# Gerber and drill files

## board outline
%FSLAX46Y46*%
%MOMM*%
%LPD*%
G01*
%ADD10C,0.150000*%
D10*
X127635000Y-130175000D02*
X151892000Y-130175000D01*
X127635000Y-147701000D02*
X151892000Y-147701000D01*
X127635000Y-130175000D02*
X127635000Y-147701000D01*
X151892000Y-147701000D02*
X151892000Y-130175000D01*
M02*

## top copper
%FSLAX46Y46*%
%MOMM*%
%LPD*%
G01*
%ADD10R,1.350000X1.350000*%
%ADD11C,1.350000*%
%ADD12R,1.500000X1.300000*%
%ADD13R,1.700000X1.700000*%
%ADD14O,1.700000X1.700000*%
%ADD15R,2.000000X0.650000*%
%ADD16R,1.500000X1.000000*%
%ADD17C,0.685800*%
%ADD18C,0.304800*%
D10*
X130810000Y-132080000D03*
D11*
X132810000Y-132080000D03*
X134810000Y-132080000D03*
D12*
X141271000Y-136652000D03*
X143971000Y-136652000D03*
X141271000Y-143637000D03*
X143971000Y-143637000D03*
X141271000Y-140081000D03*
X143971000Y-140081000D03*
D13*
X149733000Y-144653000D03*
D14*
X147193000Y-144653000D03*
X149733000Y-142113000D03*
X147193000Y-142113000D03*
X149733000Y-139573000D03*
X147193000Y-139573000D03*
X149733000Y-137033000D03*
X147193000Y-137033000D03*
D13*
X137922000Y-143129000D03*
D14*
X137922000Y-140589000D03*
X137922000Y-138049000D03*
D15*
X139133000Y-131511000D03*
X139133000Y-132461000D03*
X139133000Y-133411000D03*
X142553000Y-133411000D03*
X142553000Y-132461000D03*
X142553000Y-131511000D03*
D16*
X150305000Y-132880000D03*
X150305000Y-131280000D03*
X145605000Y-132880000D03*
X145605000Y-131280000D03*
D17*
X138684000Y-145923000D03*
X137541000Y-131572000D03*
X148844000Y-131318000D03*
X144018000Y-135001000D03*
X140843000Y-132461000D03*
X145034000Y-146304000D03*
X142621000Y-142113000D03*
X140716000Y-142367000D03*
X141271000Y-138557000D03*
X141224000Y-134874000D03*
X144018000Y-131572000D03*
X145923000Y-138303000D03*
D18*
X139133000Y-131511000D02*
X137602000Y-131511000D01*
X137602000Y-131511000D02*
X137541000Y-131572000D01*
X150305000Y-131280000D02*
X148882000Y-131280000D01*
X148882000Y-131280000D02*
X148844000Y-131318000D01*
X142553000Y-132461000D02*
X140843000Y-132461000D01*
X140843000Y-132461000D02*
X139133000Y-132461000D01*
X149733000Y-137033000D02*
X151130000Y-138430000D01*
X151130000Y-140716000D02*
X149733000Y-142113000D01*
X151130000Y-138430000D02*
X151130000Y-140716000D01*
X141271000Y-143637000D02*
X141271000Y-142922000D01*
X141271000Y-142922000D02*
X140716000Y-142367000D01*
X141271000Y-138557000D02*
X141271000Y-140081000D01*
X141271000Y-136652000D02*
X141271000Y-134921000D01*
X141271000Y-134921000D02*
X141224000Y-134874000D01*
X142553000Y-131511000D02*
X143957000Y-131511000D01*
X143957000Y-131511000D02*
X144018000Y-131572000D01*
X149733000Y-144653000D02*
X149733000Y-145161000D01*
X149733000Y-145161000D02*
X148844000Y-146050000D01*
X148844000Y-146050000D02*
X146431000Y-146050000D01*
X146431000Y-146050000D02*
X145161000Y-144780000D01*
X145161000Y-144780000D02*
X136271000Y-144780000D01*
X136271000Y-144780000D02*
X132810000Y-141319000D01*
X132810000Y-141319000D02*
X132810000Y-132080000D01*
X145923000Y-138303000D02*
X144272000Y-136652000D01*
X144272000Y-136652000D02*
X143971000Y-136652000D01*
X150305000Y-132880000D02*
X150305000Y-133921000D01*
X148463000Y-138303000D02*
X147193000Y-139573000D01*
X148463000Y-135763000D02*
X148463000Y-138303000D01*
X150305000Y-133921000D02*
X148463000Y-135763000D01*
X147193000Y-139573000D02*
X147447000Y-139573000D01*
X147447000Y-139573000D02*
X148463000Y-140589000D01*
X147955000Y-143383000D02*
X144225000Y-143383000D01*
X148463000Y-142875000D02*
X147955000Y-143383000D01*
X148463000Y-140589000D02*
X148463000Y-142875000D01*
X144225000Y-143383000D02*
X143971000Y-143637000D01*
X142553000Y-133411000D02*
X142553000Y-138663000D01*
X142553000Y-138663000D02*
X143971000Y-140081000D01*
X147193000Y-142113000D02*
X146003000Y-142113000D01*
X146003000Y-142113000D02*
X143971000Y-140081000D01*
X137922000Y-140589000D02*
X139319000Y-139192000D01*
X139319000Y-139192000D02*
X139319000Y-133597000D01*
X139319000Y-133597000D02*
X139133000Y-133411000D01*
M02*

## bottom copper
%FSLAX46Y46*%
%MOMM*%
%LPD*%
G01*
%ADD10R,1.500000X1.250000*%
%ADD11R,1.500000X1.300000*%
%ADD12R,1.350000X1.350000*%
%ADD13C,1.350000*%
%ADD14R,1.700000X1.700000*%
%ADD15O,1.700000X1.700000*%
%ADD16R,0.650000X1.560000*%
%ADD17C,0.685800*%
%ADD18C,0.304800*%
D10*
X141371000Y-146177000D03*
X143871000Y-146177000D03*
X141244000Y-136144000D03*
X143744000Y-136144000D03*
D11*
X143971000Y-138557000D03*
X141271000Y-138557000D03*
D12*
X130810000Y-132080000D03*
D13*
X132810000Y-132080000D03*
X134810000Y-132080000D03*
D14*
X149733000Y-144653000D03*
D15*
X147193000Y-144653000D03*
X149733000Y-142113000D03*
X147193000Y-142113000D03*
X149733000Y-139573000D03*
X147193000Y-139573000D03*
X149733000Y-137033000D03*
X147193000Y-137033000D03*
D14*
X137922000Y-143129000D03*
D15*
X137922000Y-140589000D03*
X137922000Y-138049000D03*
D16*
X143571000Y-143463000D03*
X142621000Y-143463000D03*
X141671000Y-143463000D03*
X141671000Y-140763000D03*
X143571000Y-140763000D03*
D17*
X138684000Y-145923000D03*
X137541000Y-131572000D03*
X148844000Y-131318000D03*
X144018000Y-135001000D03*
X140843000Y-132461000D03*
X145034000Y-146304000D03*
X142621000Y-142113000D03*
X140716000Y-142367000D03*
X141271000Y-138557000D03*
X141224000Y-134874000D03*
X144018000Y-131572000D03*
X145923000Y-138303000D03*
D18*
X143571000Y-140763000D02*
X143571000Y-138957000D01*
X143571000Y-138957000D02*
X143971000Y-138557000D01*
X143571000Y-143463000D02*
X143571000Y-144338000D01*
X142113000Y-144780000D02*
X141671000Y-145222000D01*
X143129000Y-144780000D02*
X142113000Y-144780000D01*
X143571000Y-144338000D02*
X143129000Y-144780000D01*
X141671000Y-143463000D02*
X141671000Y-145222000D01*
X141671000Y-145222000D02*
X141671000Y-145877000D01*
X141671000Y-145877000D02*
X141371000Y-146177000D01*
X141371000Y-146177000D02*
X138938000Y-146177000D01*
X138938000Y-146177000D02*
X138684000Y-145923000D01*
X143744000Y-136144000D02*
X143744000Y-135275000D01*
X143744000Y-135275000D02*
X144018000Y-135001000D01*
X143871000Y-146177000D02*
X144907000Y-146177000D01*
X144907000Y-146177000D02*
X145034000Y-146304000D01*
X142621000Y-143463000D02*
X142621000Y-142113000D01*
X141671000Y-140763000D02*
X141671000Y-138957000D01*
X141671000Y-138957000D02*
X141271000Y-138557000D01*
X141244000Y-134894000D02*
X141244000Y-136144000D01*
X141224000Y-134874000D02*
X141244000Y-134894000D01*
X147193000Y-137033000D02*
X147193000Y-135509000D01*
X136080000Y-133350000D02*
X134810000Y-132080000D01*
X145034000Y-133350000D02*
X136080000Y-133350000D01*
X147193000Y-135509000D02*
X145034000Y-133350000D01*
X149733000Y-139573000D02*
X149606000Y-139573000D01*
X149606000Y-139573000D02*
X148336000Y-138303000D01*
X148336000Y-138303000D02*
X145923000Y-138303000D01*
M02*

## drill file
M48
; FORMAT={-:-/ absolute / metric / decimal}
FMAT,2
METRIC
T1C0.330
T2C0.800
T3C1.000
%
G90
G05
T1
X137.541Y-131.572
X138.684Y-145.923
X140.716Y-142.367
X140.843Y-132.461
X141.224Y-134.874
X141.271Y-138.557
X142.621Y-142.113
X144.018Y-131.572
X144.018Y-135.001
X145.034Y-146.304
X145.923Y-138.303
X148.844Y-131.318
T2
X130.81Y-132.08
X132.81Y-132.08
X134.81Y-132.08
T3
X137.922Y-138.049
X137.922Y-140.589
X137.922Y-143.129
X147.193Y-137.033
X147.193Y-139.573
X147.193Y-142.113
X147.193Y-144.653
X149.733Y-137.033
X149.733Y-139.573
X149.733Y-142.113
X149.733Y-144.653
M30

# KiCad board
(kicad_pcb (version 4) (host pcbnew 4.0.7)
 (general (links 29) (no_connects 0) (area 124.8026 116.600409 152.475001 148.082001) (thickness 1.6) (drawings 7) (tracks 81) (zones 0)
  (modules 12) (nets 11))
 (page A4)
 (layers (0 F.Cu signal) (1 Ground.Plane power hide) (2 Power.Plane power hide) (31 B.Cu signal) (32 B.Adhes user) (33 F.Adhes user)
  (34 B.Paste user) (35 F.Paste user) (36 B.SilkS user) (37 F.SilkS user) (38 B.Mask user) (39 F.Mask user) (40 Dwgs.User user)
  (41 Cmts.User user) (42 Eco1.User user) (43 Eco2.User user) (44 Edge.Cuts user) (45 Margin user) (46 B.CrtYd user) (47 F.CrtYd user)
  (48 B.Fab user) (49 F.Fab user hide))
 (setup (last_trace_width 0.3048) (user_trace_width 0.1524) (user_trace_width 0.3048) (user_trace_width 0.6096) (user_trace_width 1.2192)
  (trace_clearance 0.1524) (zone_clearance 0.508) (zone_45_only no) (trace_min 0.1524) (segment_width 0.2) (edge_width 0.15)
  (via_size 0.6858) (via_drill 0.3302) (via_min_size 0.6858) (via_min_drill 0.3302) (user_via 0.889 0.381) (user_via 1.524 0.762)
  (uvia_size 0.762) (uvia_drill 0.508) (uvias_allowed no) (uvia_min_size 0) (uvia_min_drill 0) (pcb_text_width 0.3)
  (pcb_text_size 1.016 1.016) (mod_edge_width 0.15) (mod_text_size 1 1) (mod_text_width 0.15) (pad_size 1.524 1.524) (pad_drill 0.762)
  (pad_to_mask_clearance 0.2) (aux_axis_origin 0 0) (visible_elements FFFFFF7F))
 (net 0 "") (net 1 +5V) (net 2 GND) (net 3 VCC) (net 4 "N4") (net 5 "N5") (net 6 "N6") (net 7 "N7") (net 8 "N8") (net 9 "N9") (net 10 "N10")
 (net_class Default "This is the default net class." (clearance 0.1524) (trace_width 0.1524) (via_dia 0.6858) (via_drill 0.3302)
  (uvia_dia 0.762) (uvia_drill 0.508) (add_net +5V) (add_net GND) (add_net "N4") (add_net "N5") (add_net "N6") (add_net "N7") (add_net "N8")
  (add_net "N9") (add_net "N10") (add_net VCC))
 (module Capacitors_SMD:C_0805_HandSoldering (layer B.Cu) (at 142.621 146.177)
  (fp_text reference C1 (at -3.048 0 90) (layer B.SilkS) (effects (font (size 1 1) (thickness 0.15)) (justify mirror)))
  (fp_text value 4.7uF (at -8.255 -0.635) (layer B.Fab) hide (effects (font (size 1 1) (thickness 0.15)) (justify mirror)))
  (pad 1 smd rect (at -1.25 0) (size 1.5 1.25) (layers B.Cu B.Paste B.Mask) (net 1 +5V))
  (pad 2 smd rect (at 1.25 0) (size 1.5 1.25) (layers B.Cu B.Paste B.Mask) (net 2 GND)))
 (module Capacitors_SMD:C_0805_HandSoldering (layer B.Cu) (at 142.494 136.144)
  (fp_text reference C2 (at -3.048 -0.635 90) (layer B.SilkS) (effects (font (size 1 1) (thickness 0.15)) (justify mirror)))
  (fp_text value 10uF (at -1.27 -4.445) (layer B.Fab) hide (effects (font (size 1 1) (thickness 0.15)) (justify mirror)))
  (pad 1 smd rect (at -1.25 0) (size 1.5 1.25) (layers B.Cu B.Paste B.Mask) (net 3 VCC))
  (pad 2 smd rect (at 1.25 0) (size 1.5 1.25) (layers B.Cu B.Paste B.Mask) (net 2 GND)))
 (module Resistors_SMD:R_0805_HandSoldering (layer B.Cu) (at 142.621 138.557 180)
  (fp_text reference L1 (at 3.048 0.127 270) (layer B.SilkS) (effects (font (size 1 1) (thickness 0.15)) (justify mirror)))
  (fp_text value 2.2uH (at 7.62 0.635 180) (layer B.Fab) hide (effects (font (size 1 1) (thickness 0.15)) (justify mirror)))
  (pad 1 smd rect (at -1.35 0 180) (size 1.5 1.3) (layers B.Cu B.Paste B.Mask) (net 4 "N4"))
  (pad 2 smd rect (at 1.35 0 180) (size 1.5 1.3) (layers B.Cu B.Paste B.Mask) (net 3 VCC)))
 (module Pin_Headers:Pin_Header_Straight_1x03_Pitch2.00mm (layer F.Cu) (at 130.81 132.08 90)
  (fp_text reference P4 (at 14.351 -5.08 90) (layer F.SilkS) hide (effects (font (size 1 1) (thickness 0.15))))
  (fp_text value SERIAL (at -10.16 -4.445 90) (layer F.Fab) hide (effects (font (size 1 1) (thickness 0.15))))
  (pad 1 thru_hole rect (at 0 0 90) (size 1.35 1.35) (drill 0.8) (layers *.Cu *.Mask) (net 2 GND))
  (pad 2 thru_hole circle (at 0 2 90) (size 1.35 1.35) (drill 0.8) (layers *.Cu *.Mask) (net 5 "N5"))
  (pad 3 thru_hole circle (at 0 4 90) (size 1.35 1.35) (drill 0.8) (layers *.Cu *.Mask) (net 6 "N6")))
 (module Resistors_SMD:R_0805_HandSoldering (layer F.Cu) (at 142.621 136.652)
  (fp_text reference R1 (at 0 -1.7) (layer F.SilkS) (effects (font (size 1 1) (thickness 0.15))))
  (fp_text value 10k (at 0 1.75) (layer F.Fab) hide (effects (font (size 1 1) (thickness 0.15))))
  (pad 1 smd rect (at -1.35 0) (size 1.5 1.3) (layers F.Cu F.Paste F.Mask) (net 3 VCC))
  (pad 2 smd rect (at 1.35 0) (size 1.5 1.3) (layers F.Cu F.Paste F.Mask) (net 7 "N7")))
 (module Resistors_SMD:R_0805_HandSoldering (layer F.Cu) (at 142.621 143.637)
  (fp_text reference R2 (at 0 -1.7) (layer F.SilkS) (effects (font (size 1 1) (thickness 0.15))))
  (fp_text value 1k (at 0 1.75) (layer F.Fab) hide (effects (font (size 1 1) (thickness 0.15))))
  (pad 1 smd rect (at -1.35 0) (size 1.5 1.3) (layers F.Cu F.Paste F.Mask) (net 3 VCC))
  (pad 2 smd rect (at 1.35 0) (size 1.5 1.3) (layers F.Cu F.Paste F.Mask) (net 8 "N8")))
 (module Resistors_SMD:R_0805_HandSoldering (layer F.Cu) (at 142.621 140.081)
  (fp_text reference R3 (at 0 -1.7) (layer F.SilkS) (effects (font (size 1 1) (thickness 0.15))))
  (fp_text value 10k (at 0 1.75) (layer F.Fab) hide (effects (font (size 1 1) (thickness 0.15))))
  (pad 1 smd rect (at -1.35 0) (size 1.5 1.3) (layers F.Cu F.Paste F.Mask) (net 3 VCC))
  (pad 2 smd rect (at 1.35 0) (size 1.5 1.3) (layers F.Cu F.Paste F.Mask) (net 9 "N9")))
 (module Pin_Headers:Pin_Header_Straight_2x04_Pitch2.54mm (layer F.Cu) (at 149.733 144.653 180)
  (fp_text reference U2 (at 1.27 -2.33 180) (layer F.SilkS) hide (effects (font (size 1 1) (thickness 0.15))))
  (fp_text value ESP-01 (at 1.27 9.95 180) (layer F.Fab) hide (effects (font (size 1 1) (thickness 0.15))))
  (pad 1 thru_hole rect (at 0 0 180) (size 1.7 1.7) (drill 1) (layers *.Cu *.Mask) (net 5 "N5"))
  (pad 2 thru_hole oval (at 2.54 0 180) (size 1.7 1.7) (drill 1) (layers *.Cu *.Mask) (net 2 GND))
  (pad 3 thru_hole oval (at 0 2.54 180) (size 1.7 1.7) (drill 1) (layers *.Cu *.Mask) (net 3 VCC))
  (pad 4 thru_hole oval (at 2.54 2.54 180) (size 1.7 1.7) (drill 1) (layers *.Cu *.Mask) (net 9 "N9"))
  (pad 5 thru_hole oval (at 0 5.08 180) (size 1.7 1.7) (drill 1) (layers *.Cu *.Mask) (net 7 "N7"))
  (pad 6 thru_hole oval (at 2.54 5.08 180) (size 1.7 1.7) (drill 1) (layers *.Cu *.Mask) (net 8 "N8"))
  (pad 7 thru_hole oval (at 0 7.62 180) (size 1.7 1.7) (drill 1) (layers *.Cu *.Mask) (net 3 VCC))
  (pad 8 thru_hole oval (at 2.54 7.62 180) (size 1.7 1.7) (drill 1) (layers *.Cu *.Mask) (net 6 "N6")))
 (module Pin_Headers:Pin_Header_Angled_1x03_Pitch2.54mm (layer F.Cu) (at 137.922 143.129 180)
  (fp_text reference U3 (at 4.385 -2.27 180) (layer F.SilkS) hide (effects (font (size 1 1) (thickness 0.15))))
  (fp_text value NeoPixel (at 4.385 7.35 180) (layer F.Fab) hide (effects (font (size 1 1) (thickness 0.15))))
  (pad 1 thru_hole rect (at 0 0 180) (size 1.7 1.7) (drill 1) (layers *.Cu *.Mask) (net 2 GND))
  (pad 2 thru_hole oval (at 0 2.54 180) (size 1.7 1.7) (drill 1) (layers *.Cu *.Mask) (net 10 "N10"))
  (pad 3 thru_hole oval (at 0 5.08 180) (size 1.7 1.7) (drill 1) (layers *.Cu *.Mask) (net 1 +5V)))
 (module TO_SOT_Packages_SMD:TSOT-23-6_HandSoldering (layer F.Cu) (at 140.843 132.461)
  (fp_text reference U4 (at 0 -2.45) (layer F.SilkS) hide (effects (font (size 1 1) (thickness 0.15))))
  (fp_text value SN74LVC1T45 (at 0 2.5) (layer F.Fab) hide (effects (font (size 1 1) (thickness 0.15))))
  (pad 1 smd rect (at -1.71 -0.95) (size 2 0.65) (layers F.Cu F.Paste F.Mask) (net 1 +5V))
  (pad 2 smd rect (at -1.71 0) (size 2 0.65) (layers F.Cu F.Paste F.Mask) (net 2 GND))
  (pad 3 smd rect (at -1.71 0.95) (size 2 0.65) (layers F.Cu F.Paste F.Mask) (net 10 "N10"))
  (pad 4 smd rect (at 1.71 0.95) (size 2 0.65) (layers F.Cu F.Paste F.Mask) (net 9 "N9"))
  (pad 5 smd rect (at 1.71 0) (size 2 0.65) (layers F.Cu F.Paste F.Mask) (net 2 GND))
  (pad 6 smd rect (at 1.71 -0.95) (size 2 0.65) (layers F.Cu F.Paste F.Mask) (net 3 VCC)))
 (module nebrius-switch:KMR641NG (layer F.Cu) (at 147.955 132.08 180)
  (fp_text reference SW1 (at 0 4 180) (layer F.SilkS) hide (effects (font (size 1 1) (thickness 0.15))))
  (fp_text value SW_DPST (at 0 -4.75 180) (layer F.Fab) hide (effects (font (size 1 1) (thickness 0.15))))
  (pad 1 smd rect (at -2.35 -0.8 180) (size 1.5 1) (layers F.Cu F.Paste F.Mask) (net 8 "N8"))
  (pad 2 smd rect (at -2.35 0.8 180) (size 1.5 1) (layers F.Cu F.Paste F.Mask) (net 2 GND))
  (pad 3 smd rect (at 2.35 -0.8 180) (size 1.5 1) (layers F.Cu F.Paste F.Mask))
  (pad 4 smd rect (at 2.35 0.8 180) (size 1.5 1) (layers F.Cu F.Paste F.Mask)))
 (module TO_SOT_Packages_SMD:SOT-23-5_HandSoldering (layer B.Cu) (at 142.621 142.113 90)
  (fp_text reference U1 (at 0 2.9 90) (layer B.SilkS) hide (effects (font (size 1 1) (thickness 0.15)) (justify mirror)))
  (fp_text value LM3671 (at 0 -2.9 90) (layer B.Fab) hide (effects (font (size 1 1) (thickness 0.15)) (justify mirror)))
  (pad 1 smd rect (at -1.35 0.95 90) (size 1.56 0.65) (layers B.Cu B.Paste B.Mask) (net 1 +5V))
  (pad 2 smd rect (at -1.35 0 90) (size 1.56 0.65) (layers B.Cu B.Paste B.Mask) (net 2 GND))
  (pad 3 smd rect (at -1.35 -0.95 90) (size 1.56 0.65) (layers B.Cu B.Paste B.Mask) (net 1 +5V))
  (pad 4 smd rect (at 1.35 -0.95 90) (size 1.56 0.65) (layers B.Cu B.Paste B.Mask) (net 3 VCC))
  (pad 5 smd rect (at 1.35 0.95 90) (size 1.56 0.65) (layers B.Cu B.Paste B.Mask) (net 4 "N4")))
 (gr_line (start 127.635 130.175) (end 151.892 130.175) (angle 90) (layer Edge.Cuts) (width 0.15))
 (gr_line (start 127.635 147.701) (end 151.892 147.701) (angle 90) (layer Edge.Cuts) (width 0.15))
 (gr_line (start 127.635 130.175) (end 127.635 147.701) (angle 90) (layer Edge.Cuts) (width 0.15))
 (gr_line (start 151.892 147.701) (end 151.892 130.175) (angle 90) (layer Edge.Cuts) (width 0.15))
 (segment (start 143.571 140.763) (end 143.571 138.957) (width 0.3048) (layer B.Cu) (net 4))
 (segment (start 143.571 138.957) (end 143.971 138.557) (width 0.3048) (layer B.Cu) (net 4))
 (segment (start 143.571 143.463) (end 143.571 144.338) (width 0.3048) (layer B.Cu) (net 1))
 (segment (start 142.113 144.78) (end 141.671 145.222) (width 0.3048) (layer B.Cu) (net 1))
 (segment (start 143.129 144.78) (end 142.113 144.78) (width 0.3048) (layer B.Cu) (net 1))
 (segment (start 143.571 144.338) (end 143.129 144.78) (width 0.3048) (layer B.Cu) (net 1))
 (segment (start 141.671 143.463) (end 141.671 145.222) (width 0.3048) (layer B.Cu) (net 1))
 (segment (start 141.671 145.222) (end 141.671 145.877) (width 0.3048) (layer B.Cu) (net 1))
 (segment (start 141.671 145.877) (end 141.371 146.177) (width 0.3048) (layer B.Cu) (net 1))
 (segment (start 141.371 146.177) (end 138.938 146.177) (width 0.3048) (layer B.Cu) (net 1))
 (via (at 138.684 145.923) (size 0.6858) (drill 0.3302) (layers F.Cu B.Cu) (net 1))
 (segment (start 138.938 146.177) (end 138.684 145.923) (width 0.3048) (layer B.Cu) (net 1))
 (segment (start 139.133 131.511) (end 137.602 131.511) (width 0.3048) (layer F.Cu) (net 1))
 (via (at 137.541 131.572) (size 0.6858) (drill 0.3302) (layers F.Cu B.Cu) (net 1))
 (segment (start 137.602 131.511) (end 137.541 131.572) (width 0.3048) (layer F.Cu) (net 1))
 (segment (start 150.305 131.28) (end 148.882 131.28) (width 0.3048) (layer F.Cu) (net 2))
 (via (at 148.844 131.318) (size 0.6858) (drill 0.3302) (layers F.Cu B.Cu) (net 2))
 (segment (start 148.882 131.28) (end 148.844 131.318) (width 0.3048) (layer F.Cu) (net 2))
 (segment (start 143.744 136.144) (end 143.744 135.275) (width 0.3048) (layer B.Cu) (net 2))
 (via (at 144.018 135.001) (size 0.6858) (drill 0.3302) (layers F.Cu B.Cu) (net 2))
 (segment (start 143.744 135.275) (end 144.018 135.001) (width 0.3048) (layer B.Cu) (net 2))
 (segment (start 142.553 132.461) (end 140.843 132.461) (width 0.3048) (layer F.Cu) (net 2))
 (via (at 140.843 132.461) (size 0.6858) (drill 0.3302) (layers F.Cu B.Cu) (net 2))
 (segment (start 140.843 132.461) (end 139.133 132.461) (width 0.3048) (layer F.Cu) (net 2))
 (segment (start 143.871 146.177) (end 144.907 146.177) (width 0.3048) (layer B.Cu) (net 2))
 (via (at 145.034 146.304) (size 0.6858) (drill 0.3302) (layers F.Cu B.Cu) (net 2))
 (segment (start 144.907 146.177) (end 145.034 146.304) (width 0.3048) (layer B.Cu) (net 2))
 (segment (start 142.621 143.463) (end 142.621 142.113) (width 0.3048) (layer B.Cu) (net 2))
 (via (at 142.621 142.113) (size 0.6858) (drill 0.3302) (layers F.Cu B.Cu) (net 2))
 (segment (start 149.733 137.033) (end 151.13 138.43) (width 0.3048) (layer F.Cu) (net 3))
 (segment (start 151.13 140.716) (end 149.733 142.113) (width 0.3048) (layer F.Cu) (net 3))
 (segment (start 151.13 138.43) (end 151.13 140.716) (width 0.3048) (layer F.Cu) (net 3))
 (segment (start 141.271 143.637) (end 141.271 142.922) (width 0.3048) (layer F.Cu) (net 3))
 (via (at 140.716 142.367) (size 0.6858) (drill 0.3302) (layers F.Cu B.Cu) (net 3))
 (segment (start 141.271 142.922) (end 140.716 142.367) (width 0.3048) (layer F.Cu) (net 3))
 (segment (start 141.671 140.763) (end 141.671 138.957) (width 0.3048) (layer B.Cu) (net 3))
 (segment (start 141.671 138.957) (end 141.271 138.557) (width 0.3048) (layer B.Cu) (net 3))
 (via (at 141.271 138.557) (size 0.6858) (drill 0.3302) (layers F.Cu B.Cu) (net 3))
 (segment (start 141.271 138.557) (end 141.271 140.081) (width 0.3048) (layer F.Cu) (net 3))
 (segment (start 141.271 136.652) (end 141.271 134.921) (width 0.3048) (layer F.Cu) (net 3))
 (segment (start 141.244 134.894) (end 141.244 136.144) (width 0.3048) (layer B.Cu) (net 3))
 (segment (start 141.224 134.874) (end 141.244 134.894) (width 0.3048) (layer B.Cu) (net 3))
 (via (at 141.224 134.874) (size 0.6858) (drill 0.3302) (layers F.Cu B.Cu) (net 3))
 (segment (start 141.271 134.921) (end 141.224 134.874) (width 0.3048) (layer F.Cu) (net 3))
 (segment (start 142.553 131.511) (end 143.957 131.511) (width 0.3048) (layer F.Cu) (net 3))
 (via (at 144.018 131.572) (size 0.6858) (drill 0.3302) (layers F.Cu B.Cu) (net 3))
 (segment (start 143.957 131.511) (end 144.018 131.572) (width 0.3048) (layer F.Cu) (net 3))
 (segment (start 149.733 144.653) (end 149.733 145.161) (width 0.3048) (layer F.Cu) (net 5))
 (segment (start 149.733 145.161) (end 148.844 146.05) (width 0.3048) (layer F.Cu) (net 5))
 (segment (start 148.844 146.05) (end 146.431 146.05) (width 0.3048) (layer F.Cu) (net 5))
 (segment (start 146.431 146.05) (end 145.161 144.78) (width 0.3048) (layer F.Cu) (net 5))
 (segment (start 145.161 144.78) (end 136.271 144.78) (width 0.3048) (layer F.Cu) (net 5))
 (segment (start 136.271 144.78) (end 132.81 141.319) (width 0.3048) (layer F.Cu) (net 5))
 (segment (start 132.81 141.319) (end 132.81 132.08) (width 0.3048) (layer F.Cu) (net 5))
 (segment (start 147.193 137.033) (end 147.193 135.509) (width 0.3048) (layer B.Cu) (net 6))
 (segment (start 136.08 133.35) (end 134.81 132.08) (width 0.3048) (layer B.Cu) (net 6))
 (segment (start 145.034 133.35) (end 136.08 133.35) (width 0.3048) (layer B.Cu) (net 6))
 (segment (start 147.193 135.509) (end 145.034 133.35) (width 0.3048) (layer B.Cu) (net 6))
 (segment (start 149.733 139.573) (end 149.606 139.573) (width 0.3048) (layer B.Cu) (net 7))
 (segment (start 149.606 139.573) (end 148.336 138.303) (width 0.3048) (layer B.Cu) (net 7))
 (segment (start 148.336 138.303) (end 145.923 138.303) (width 0.3048) (layer B.Cu) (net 7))
 (via (at 145.923 138.303) (size 0.6858) (drill 0.3302) (layers F.Cu B.Cu) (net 7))
 (segment (start 145.923 138.303) (end 144.272 136.652) (width 0.3048) (layer F.Cu) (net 7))
 (segment (start 144.272 136.652) (end 143.971 136.652) (width 0.3048) (layer F.Cu) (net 7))
 (segment (start 150.305 132.88) (end 150.305 133.921) (width 0.3048) (layer F.Cu) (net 8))
 (segment (start 148.463 138.303) (end 147.193 139.573) (width 0.3048) (layer F.Cu) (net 8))
 (segment (start 148.463 135.763) (end 148.463 138.303) (width 0.3048) (layer F.Cu) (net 8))
 (segment (start 150.305 133.921) (end 148.463 135.763) (width 0.3048) (layer F.Cu) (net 8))
 (segment (start 147.193 139.573) (end 147.447 139.573) (width 0.3048) (layer F.Cu) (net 8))
 (segment (start 147.447 139.573) (end 148.463 140.589) (width 0.3048) (layer F.Cu) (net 8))
 (segment (start 147.955 143.383) (end 144.225 143.383) (width 0.3048) (layer F.Cu) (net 8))
 (segment (start 148.463 142.875) (end 147.955 143.383) (width 0.3048) (layer F.Cu) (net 8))
 (segment (start 148.463 140.589) (end 148.463 142.875) (width 0.3048) (layer F.Cu) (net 8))
 (segment (start 144.225 143.383) (end 143.971 143.637) (width 0.3048) (layer F.Cu) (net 8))
 (segment (start 142.553 133.411) (end 142.553 138.663) (width 0.3048) (layer F.Cu) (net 9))
 (segment (start 142.553 138.663) (end 143.971 140.081) (width 0.3048) (layer F.Cu) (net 9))
 (segment (start 147.193 142.113) (end 146.003 142.113) (width 0.3048) (layer F.Cu) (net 9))
 (segment (start 146.003 142.113) (end 143.971 140.081) (width 0.3048) (layer F.Cu) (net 9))
 (segment (start 137.922 140.589) (end 139.319 139.192) (width 0.3048) (layer F.Cu) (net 10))
 (segment (start 139.319 139.192) (end 139.319 133.597) (width 0.3048) (layer F.Cu) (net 10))
 (segment (start 139.319 133.597) (end 139.133 133.411) (width 0.3048) (layer F.Cu) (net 10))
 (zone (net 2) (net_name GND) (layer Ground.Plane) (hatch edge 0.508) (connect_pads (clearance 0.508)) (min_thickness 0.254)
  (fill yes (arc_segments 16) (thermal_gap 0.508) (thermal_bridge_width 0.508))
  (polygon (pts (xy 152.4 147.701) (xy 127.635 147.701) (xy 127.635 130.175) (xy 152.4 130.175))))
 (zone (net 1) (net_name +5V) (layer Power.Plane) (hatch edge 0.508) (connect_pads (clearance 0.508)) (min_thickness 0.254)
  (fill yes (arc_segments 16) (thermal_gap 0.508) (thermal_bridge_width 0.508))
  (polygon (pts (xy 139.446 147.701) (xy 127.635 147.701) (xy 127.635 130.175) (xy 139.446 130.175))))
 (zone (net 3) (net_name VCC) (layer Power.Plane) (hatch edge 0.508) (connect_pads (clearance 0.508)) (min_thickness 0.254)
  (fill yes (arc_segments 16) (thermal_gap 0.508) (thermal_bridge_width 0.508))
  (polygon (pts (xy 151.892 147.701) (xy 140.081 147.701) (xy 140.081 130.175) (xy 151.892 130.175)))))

